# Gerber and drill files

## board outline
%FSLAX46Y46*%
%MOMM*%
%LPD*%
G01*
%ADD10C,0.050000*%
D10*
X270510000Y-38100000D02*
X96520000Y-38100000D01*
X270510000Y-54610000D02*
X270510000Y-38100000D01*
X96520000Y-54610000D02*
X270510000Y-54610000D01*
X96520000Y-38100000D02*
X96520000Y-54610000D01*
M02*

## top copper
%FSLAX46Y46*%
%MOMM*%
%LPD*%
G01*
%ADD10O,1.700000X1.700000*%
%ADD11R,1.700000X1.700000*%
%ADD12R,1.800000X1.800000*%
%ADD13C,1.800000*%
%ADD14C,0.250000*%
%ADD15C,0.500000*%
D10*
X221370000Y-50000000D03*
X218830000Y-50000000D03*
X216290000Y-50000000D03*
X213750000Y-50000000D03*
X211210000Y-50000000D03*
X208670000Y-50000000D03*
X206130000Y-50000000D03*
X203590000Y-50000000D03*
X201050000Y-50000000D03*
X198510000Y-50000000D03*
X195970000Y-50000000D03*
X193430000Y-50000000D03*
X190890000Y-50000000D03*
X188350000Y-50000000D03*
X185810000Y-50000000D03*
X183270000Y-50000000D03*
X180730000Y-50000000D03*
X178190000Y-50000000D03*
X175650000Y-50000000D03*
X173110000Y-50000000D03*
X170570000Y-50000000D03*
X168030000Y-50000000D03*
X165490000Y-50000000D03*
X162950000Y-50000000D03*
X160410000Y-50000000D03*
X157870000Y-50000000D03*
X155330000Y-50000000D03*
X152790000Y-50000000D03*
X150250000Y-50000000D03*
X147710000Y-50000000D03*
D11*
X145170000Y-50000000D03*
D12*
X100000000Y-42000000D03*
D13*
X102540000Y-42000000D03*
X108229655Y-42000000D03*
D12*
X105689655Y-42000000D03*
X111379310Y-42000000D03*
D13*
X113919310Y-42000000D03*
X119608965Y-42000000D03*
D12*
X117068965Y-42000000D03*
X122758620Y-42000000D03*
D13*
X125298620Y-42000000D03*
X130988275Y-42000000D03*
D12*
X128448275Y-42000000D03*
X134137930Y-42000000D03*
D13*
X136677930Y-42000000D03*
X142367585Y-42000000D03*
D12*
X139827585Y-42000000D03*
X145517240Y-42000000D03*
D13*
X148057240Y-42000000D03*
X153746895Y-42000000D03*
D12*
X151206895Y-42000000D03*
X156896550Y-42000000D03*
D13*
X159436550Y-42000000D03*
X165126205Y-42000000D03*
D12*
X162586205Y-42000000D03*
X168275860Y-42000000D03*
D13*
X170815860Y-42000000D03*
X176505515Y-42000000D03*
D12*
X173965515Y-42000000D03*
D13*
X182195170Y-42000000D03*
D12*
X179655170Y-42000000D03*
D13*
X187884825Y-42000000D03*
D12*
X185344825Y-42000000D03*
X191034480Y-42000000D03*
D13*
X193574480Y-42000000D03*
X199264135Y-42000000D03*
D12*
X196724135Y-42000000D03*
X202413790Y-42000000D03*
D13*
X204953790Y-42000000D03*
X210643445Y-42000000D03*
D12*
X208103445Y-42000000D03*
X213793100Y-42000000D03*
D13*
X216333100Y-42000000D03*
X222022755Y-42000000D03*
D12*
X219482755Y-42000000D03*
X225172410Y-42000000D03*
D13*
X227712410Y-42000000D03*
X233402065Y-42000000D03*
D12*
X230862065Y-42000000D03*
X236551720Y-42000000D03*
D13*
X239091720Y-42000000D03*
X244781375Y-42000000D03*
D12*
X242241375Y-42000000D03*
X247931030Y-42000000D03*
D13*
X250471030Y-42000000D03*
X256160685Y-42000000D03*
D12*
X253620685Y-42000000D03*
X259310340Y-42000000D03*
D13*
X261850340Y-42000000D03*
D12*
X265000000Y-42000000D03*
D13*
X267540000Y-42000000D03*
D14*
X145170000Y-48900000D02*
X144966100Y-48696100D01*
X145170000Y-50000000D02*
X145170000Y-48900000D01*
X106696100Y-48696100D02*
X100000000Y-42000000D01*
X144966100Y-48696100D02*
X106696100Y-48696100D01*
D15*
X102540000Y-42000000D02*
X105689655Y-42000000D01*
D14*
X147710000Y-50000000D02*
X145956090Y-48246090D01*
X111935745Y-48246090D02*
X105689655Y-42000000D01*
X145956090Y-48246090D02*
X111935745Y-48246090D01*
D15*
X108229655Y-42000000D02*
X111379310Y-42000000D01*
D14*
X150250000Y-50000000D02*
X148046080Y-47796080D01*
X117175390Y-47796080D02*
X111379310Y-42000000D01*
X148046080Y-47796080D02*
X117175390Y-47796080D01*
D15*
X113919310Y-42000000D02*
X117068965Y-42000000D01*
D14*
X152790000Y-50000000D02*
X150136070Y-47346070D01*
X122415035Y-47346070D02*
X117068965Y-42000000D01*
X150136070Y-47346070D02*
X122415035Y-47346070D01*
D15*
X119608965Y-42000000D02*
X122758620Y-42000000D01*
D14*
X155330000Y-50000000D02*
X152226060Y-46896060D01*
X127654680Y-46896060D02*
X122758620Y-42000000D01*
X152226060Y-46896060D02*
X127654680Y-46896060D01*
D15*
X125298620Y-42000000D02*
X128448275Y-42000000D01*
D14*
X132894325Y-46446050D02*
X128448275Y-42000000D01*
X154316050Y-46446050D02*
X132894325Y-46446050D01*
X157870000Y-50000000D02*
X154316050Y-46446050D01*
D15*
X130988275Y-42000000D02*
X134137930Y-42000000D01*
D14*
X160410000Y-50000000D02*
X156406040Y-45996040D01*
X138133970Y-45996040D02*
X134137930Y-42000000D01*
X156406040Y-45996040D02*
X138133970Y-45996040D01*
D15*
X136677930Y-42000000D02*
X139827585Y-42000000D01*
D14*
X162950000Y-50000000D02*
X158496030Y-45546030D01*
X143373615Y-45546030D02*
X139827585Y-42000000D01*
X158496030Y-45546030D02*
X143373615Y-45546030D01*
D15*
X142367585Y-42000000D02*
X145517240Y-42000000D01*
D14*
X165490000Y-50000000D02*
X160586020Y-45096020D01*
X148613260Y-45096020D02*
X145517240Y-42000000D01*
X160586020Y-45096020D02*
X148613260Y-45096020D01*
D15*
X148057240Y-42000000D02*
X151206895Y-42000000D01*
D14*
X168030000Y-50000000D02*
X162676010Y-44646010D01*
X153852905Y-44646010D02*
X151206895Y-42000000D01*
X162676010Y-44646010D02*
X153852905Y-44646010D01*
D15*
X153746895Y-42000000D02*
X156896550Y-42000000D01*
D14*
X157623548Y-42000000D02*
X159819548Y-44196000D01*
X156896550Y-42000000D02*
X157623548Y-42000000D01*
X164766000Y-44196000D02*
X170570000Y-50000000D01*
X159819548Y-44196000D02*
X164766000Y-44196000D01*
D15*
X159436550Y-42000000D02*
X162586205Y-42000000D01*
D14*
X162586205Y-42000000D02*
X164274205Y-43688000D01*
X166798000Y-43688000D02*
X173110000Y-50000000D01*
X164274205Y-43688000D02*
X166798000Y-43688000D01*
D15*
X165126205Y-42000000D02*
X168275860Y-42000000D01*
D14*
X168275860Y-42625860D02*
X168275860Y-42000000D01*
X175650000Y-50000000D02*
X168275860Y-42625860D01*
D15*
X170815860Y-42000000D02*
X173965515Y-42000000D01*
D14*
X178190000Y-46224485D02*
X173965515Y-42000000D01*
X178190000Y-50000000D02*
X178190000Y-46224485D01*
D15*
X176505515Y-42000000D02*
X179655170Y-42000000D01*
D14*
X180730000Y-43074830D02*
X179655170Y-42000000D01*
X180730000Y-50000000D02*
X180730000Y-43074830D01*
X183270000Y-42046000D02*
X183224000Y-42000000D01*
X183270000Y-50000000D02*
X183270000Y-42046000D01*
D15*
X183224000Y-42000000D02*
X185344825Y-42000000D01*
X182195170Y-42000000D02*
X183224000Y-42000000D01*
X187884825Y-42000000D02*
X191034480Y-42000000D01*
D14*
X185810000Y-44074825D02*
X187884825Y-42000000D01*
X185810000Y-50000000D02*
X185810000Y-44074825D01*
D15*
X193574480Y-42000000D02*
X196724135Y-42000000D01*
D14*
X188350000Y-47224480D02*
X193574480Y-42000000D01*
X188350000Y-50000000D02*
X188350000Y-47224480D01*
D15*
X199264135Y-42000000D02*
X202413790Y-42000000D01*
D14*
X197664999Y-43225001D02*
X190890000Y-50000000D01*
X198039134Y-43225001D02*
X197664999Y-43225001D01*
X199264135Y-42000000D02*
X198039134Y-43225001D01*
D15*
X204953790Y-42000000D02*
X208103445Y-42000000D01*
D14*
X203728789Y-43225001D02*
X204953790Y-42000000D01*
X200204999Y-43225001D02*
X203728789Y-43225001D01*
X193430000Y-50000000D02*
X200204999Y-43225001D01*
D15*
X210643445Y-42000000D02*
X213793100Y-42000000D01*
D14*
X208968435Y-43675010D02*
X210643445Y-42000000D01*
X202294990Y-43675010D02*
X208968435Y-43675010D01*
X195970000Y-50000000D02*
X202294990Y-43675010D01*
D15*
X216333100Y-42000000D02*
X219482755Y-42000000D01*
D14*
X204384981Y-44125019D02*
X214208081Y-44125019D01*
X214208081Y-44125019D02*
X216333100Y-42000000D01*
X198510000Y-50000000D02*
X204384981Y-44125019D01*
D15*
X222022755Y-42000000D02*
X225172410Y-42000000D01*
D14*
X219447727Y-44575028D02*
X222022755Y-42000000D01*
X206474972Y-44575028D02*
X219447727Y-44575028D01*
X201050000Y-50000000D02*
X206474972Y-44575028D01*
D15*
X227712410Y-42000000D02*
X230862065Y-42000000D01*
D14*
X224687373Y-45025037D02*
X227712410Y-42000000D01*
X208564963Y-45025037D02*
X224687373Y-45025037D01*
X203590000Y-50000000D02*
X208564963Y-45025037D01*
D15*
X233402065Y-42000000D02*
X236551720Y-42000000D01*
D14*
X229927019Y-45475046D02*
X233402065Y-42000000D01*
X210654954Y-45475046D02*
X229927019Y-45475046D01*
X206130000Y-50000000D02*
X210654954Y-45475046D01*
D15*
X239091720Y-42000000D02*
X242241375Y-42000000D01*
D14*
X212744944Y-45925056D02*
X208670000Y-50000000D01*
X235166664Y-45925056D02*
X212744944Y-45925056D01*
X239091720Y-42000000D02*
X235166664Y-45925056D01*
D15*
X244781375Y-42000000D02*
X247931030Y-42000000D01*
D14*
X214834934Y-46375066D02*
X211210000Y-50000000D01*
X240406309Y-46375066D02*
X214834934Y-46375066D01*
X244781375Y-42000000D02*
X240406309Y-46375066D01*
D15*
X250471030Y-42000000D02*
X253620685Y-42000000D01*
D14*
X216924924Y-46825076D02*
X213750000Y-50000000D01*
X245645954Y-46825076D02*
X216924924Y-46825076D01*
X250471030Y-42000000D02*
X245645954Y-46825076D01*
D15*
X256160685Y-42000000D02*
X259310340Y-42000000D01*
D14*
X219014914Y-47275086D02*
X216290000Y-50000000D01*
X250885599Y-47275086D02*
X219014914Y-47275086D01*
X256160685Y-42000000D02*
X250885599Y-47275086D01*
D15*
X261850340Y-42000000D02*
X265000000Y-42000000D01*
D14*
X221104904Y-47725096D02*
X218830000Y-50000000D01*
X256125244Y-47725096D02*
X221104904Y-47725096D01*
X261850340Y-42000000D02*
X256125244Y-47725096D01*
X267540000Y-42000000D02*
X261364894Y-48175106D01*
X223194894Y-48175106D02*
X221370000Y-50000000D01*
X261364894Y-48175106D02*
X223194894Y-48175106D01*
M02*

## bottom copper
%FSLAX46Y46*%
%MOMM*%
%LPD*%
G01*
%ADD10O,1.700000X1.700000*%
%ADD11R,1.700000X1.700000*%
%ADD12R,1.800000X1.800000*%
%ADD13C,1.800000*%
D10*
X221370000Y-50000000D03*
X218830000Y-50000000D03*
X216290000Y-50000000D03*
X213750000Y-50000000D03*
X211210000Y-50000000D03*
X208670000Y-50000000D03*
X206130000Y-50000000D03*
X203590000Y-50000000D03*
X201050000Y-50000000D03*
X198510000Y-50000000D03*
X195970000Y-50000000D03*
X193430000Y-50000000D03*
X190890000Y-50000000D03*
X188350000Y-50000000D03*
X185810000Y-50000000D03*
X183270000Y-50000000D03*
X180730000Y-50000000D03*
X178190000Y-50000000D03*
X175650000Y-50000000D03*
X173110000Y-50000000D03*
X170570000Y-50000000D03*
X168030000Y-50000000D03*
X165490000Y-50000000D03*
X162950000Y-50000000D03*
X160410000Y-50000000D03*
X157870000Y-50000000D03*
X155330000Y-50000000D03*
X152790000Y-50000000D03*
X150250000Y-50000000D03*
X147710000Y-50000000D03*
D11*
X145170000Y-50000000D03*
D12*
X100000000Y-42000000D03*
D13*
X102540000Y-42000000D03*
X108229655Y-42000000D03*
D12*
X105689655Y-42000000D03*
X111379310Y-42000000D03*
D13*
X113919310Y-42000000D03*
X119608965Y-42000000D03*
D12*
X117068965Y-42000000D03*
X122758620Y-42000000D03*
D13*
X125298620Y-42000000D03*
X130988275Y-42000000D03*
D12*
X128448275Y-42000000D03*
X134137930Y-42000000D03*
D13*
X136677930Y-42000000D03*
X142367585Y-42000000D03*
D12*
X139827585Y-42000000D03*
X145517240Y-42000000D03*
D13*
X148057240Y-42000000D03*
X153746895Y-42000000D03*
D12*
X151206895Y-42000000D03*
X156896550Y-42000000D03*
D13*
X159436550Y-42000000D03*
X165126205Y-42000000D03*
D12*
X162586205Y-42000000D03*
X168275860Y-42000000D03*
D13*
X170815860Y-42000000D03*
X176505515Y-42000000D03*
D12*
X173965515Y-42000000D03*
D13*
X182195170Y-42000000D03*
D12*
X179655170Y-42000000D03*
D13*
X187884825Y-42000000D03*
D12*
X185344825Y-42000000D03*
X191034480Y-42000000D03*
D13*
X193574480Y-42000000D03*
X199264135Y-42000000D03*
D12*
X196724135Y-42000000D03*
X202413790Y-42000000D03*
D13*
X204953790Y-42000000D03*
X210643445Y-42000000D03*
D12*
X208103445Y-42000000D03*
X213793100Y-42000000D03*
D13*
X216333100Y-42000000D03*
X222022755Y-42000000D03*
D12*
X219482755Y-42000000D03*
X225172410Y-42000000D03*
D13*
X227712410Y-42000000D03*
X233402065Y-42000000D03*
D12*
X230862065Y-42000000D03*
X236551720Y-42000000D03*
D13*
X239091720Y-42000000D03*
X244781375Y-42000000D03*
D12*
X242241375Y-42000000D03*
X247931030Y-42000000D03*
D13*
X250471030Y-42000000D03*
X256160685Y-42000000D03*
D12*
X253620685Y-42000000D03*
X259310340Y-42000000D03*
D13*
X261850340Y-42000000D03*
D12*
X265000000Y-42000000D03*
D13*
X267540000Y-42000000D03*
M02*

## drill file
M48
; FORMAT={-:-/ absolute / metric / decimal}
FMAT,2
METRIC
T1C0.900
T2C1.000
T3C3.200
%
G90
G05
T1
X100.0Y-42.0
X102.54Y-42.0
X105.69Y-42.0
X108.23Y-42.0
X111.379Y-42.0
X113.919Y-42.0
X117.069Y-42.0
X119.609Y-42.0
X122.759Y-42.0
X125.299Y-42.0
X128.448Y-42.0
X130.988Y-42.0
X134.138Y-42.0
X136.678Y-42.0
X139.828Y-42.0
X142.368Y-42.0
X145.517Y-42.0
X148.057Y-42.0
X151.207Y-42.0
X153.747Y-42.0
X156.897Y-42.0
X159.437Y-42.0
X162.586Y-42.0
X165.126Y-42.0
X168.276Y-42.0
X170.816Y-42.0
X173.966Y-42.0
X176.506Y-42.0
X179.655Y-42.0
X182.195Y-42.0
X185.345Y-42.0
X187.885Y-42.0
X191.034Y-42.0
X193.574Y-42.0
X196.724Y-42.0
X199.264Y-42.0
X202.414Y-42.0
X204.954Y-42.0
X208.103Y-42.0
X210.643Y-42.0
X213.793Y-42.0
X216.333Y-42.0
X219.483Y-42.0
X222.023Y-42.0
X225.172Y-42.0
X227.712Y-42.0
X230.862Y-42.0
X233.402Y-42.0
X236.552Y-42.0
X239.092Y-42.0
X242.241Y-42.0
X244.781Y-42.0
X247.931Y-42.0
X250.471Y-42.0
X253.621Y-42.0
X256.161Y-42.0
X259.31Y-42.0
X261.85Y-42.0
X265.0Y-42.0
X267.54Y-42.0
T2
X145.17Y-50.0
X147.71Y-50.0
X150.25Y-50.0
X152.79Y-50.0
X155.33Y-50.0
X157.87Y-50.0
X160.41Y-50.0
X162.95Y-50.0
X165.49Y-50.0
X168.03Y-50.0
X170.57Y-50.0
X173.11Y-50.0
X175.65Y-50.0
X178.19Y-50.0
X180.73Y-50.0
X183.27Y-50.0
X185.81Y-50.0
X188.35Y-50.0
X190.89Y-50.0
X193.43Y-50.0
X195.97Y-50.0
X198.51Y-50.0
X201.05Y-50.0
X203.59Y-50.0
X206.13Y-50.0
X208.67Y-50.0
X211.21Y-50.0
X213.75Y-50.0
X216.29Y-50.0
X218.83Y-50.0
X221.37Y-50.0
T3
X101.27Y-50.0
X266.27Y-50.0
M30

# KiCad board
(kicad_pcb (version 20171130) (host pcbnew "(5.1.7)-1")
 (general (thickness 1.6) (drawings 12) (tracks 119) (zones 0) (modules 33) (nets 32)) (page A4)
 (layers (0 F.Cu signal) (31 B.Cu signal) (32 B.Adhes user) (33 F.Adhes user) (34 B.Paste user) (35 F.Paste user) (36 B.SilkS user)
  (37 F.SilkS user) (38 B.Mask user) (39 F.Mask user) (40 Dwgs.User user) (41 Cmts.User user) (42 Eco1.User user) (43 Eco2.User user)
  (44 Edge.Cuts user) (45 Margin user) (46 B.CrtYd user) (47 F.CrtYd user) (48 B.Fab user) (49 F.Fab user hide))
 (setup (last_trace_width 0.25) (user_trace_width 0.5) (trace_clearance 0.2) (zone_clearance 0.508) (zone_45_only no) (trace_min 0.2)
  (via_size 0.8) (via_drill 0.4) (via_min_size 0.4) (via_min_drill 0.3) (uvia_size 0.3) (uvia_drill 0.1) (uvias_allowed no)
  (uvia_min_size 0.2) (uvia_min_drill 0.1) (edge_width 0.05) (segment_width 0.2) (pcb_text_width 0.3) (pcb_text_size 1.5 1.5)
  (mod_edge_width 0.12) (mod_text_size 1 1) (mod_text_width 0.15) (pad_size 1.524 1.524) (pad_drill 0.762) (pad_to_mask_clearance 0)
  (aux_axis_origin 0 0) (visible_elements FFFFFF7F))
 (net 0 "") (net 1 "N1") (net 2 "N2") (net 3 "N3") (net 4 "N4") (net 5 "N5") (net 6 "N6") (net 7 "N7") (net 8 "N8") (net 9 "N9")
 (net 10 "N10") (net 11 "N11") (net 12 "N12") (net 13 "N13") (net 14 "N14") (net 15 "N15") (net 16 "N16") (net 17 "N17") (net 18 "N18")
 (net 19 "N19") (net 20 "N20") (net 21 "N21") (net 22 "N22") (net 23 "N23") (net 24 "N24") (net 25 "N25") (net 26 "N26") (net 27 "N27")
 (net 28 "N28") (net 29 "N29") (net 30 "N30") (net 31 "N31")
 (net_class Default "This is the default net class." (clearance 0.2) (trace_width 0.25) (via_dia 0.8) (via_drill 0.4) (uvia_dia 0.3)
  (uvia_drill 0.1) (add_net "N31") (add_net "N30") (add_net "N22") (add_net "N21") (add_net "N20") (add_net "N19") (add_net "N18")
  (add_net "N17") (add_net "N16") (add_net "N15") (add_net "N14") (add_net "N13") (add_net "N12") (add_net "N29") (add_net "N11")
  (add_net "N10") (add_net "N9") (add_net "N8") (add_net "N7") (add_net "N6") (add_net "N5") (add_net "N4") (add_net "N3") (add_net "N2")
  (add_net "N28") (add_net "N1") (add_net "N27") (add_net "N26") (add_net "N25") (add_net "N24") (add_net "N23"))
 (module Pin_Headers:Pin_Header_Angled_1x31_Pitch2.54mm (layer F.Cu) (at 145.17 50 90)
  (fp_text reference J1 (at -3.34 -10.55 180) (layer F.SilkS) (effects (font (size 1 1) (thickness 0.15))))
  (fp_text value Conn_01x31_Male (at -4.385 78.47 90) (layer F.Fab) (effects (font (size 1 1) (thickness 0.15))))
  (pad 31 thru_hole oval (at 0 76.2 90) (size 1.7 1.7) (drill 1) (layers *.Cu *.Mask) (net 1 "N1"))
  (pad 30 thru_hole oval (at 0 73.66 90) (size 1.7 1.7) (drill 1) (layers *.Cu *.Mask) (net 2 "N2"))
  (pad 29 thru_hole oval (at 0 71.12 90) (size 1.7 1.7) (drill 1) (layers *.Cu *.Mask) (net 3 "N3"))
  (pad 28 thru_hole oval (at 0 68.58 90) (size 1.7 1.7) (drill 1) (layers *.Cu *.Mask) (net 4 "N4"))
  (pad 27 thru_hole oval (at 0 66.04 90) (size 1.7 1.7) (drill 1) (layers *.Cu *.Mask) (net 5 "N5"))
  (pad 26 thru_hole oval (at 0 63.5 90) (size 1.7 1.7) (drill 1) (layers *.Cu *.Mask) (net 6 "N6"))
  (pad 25 thru_hole oval (at 0 60.96 90) (size 1.7 1.7) (drill 1) (layers *.Cu *.Mask) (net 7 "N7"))
  (pad 24 thru_hole oval (at 0 58.42 90) (size 1.7 1.7) (drill 1) (layers *.Cu *.Mask) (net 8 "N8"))
  (pad 23 thru_hole oval (at 0 55.88 90) (size 1.7 1.7) (drill 1) (layers *.Cu *.Mask) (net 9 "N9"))
  (pad 22 thru_hole oval (at 0 53.34 90) (size 1.7 1.7) (drill 1) (layers *.Cu *.Mask) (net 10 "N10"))
  (pad 21 thru_hole oval (at 0 50.8 90) (size 1.7 1.7) (drill 1) (layers *.Cu *.Mask) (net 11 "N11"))
  (pad 20 thru_hole oval (at 0 48.26 90) (size 1.7 1.7) (drill 1) (layers *.Cu *.Mask) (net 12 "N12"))
  (pad 19 thru_hole oval (at 0 45.72 90) (size 1.7 1.7) (drill 1) (layers *.Cu *.Mask) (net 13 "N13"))
  (pad 18 thru_hole oval (at 0 43.18 90) (size 1.7 1.7) (drill 1) (layers *.Cu *.Mask) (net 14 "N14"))
  (pad 17 thru_hole oval (at 0 40.64 90) (size 1.7 1.7) (drill 1) (layers *.Cu *.Mask) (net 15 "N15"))
  (pad 16 thru_hole oval (at 0 38.1 90) (size 1.7 1.7) (drill 1) (layers *.Cu *.Mask) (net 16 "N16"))
  (pad 15 thru_hole oval (at 0 35.56 90) (size 1.7 1.7) (drill 1) (layers *.Cu *.Mask) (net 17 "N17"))
  (pad 14 thru_hole oval (at 0 33.02 90) (size 1.7 1.7) (drill 1) (layers *.Cu *.Mask) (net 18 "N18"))
  (pad 13 thru_hole oval (at 0 30.48 90) (size 1.7 1.7) (drill 1) (layers *.Cu *.Mask) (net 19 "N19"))
  (pad 12 thru_hole oval (at 0 27.94 90) (size 1.7 1.7) (drill 1) (layers *.Cu *.Mask) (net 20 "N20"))
  (pad 11 thru_hole oval (at 0 25.4 90) (size 1.7 1.7) (drill 1) (layers *.Cu *.Mask) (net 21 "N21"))
  (pad 10 thru_hole oval (at 0 22.86 90) (size 1.7 1.7) (drill 1) (layers *.Cu *.Mask) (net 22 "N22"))
  (pad 9 thru_hole oval (at 0 20.32 90) (size 1.7 1.7) (drill 1) (layers *.Cu *.Mask) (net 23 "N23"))
  (pad 8 thru_hole oval (at 0 17.78 90) (size 1.7 1.7) (drill 1) (layers *.Cu *.Mask) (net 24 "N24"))
  (pad 7 thru_hole oval (at 0 15.24 90) (size 1.7 1.7) (drill 1) (layers *.Cu *.Mask) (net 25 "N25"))
  (pad 6 thru_hole oval (at 0 12.7 90) (size 1.7 1.7) (drill 1) (layers *.Cu *.Mask) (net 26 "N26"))
  (pad 5 thru_hole oval (at 0 10.16 90) (size 1.7 1.7) (drill 1) (layers *.Cu *.Mask) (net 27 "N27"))
  (pad 4 thru_hole oval (at 0 7.62 90) (size 1.7 1.7) (drill 1) (layers *.Cu *.Mask) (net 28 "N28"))
  (pad 3 thru_hole oval (at 0 5.08 90) (size 1.7 1.7) (drill 1) (layers *.Cu *.Mask) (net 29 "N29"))
  (pad 2 thru_hole oval (at 0 2.54 90) (size 1.7 1.7) (drill 1) (layers *.Cu *.Mask) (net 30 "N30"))
  (pad 1 thru_hole rect (at 0 0 90) (size 1.7 1.7) (drill 1) (layers *.Cu *.Mask) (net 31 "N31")))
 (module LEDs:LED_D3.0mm (layer F.Cu) (at 100 42)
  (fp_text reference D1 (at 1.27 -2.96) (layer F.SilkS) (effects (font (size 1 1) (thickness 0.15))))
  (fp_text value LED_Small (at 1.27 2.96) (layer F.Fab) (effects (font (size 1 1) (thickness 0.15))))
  (pad 1 thru_hole rect (at 0 0) (size 1.8 1.8) (drill 0.9) (layers *.Cu *.Mask) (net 31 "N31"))
  (pad 2 thru_hole circle (at 2.54 0) (size 1.8 1.8) (drill 0.9) (layers *.Cu *.Mask) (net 30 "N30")))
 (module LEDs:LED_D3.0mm (layer F.Cu) (at 105.689655 42)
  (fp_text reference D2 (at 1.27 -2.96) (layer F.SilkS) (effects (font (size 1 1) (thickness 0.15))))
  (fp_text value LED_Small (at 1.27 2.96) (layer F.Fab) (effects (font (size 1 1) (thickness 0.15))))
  (pad 2 thru_hole circle (at 2.54 0) (size 1.8 1.8) (drill 0.9) (layers *.Cu *.Mask) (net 29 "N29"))
  (pad 1 thru_hole rect (at 0 0) (size 1.8 1.8) (drill 0.9) (layers *.Cu *.Mask) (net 30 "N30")))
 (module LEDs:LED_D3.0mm (layer F.Cu) (at 111.37931 42)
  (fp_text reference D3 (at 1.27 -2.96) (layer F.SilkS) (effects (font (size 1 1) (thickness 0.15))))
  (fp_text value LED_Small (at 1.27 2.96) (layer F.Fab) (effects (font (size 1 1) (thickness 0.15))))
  (pad 1 thru_hole rect (at 0 0) (size 1.8 1.8) (drill 0.9) (layers *.Cu *.Mask) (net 29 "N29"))
  (pad 2 thru_hole circle (at 2.54 0) (size 1.8 1.8) (drill 0.9) (layers *.Cu *.Mask) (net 28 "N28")))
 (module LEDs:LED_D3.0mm (layer F.Cu) (at 117.068965 42)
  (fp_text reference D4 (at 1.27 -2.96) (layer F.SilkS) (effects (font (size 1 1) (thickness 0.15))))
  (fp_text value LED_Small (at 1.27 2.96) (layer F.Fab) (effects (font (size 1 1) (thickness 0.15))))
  (pad 2 thru_hole circle (at 2.54 0) (size 1.8 1.8) (drill 0.9) (layers *.Cu *.Mask) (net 27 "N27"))
  (pad 1 thru_hole rect (at 0 0) (size 1.8 1.8) (drill 0.9) (layers *.Cu *.Mask) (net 28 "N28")))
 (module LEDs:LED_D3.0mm (layer F.Cu) (at 122.75862 42)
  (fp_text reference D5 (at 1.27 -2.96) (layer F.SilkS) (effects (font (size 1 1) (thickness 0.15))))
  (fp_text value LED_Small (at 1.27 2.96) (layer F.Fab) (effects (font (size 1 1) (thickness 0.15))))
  (pad 1 thru_hole rect (at 0 0) (size 1.8 1.8) (drill 0.9) (layers *.Cu *.Mask) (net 27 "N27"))
  (pad 2 thru_hole circle (at 2.54 0) (size 1.8 1.8) (drill 0.9) (layers *.Cu *.Mask) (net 26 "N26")))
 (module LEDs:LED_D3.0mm (layer F.Cu) (at 128.448275 42)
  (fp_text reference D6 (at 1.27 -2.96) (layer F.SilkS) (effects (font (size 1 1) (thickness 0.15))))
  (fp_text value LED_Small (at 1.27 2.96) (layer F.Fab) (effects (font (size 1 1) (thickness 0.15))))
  (pad 2 thru_hole circle (at 2.54 0) (size 1.8 1.8) (drill 0.9) (layers *.Cu *.Mask) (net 25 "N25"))
  (pad 1 thru_hole rect (at 0 0) (size 1.8 1.8) (drill 0.9) (layers *.Cu *.Mask) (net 26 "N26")))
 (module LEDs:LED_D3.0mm (layer F.Cu) (at 134.13793 42)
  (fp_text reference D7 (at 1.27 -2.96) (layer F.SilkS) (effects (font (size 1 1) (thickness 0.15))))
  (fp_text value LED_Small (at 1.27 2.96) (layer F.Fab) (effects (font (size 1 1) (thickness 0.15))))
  (pad 1 thru_hole rect (at 0 0) (size 1.8 1.8) (drill 0.9) (layers *.Cu *.Mask) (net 25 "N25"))
  (pad 2 thru_hole circle (at 2.54 0) (size 1.8 1.8) (drill 0.9) (layers *.Cu *.Mask) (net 24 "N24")))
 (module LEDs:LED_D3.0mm (layer F.Cu) (at 139.827585 42)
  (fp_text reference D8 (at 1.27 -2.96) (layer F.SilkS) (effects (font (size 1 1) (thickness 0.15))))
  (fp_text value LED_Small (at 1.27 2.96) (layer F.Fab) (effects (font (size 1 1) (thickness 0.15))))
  (pad 2 thru_hole circle (at 2.54 0) (size 1.8 1.8) (drill 0.9) (layers *.Cu *.Mask) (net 23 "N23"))
  (pad 1 thru_hole rect (at 0 0) (size 1.8 1.8) (drill 0.9) (layers *.Cu *.Mask) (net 24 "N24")))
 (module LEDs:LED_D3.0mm (layer F.Cu) (at 145.51724 42)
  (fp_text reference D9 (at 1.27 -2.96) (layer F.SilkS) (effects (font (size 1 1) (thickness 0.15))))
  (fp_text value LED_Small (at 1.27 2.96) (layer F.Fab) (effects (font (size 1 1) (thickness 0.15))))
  (pad 1 thru_hole rect (at 0 0) (size 1.8 1.8) (drill 0.9) (layers *.Cu *.Mask) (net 23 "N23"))
  (pad 2 thru_hole circle (at 2.54 0) (size 1.8 1.8) (drill 0.9) (layers *.Cu *.Mask) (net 22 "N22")))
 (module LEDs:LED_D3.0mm (layer F.Cu) (at 151.206895 42)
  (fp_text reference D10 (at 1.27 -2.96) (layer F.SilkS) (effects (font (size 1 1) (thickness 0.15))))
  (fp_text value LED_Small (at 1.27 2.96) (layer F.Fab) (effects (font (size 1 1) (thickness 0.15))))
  (pad 2 thru_hole circle (at 2.54 0) (size 1.8 1.8) (drill 0.9) (layers *.Cu *.Mask) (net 21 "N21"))
  (pad 1 thru_hole rect (at 0 0) (size 1.8 1.8) (drill 0.9) (layers *.Cu *.Mask) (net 22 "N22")))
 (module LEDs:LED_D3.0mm (layer F.Cu) (at 156.89655 42)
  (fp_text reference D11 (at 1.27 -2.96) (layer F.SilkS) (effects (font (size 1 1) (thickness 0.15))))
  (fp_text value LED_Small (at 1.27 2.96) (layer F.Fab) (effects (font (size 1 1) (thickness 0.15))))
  (pad 1 thru_hole rect (at 0 0) (size 1.8 1.8) (drill 0.9) (layers *.Cu *.Mask) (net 21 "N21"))
  (pad 2 thru_hole circle (at 2.54 0) (size 1.8 1.8) (drill 0.9) (layers *.Cu *.Mask) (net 20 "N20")))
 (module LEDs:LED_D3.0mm (layer F.Cu) (at 162.586205 42)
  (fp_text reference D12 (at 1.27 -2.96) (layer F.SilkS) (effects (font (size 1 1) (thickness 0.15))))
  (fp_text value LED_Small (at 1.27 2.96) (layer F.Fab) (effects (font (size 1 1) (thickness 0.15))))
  (pad 2 thru_hole circle (at 2.54 0) (size 1.8 1.8) (drill 0.9) (layers *.Cu *.Mask) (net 19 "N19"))
  (pad 1 thru_hole rect (at 0 0) (size 1.8 1.8) (drill 0.9) (layers *.Cu *.Mask) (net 20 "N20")))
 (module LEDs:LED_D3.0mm (layer F.Cu) (at 168.27586 42)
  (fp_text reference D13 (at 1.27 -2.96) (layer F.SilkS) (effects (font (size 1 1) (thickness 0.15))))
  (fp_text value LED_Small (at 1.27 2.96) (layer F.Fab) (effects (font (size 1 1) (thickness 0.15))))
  (pad 1 thru_hole rect (at 0 0) (size 1.8 1.8) (drill 0.9) (layers *.Cu *.Mask) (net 19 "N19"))
  (pad 2 thru_hole circle (at 2.54 0) (size 1.8 1.8) (drill 0.9) (layers *.Cu *.Mask) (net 18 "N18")))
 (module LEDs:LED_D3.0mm (layer F.Cu) (at 173.965515 42)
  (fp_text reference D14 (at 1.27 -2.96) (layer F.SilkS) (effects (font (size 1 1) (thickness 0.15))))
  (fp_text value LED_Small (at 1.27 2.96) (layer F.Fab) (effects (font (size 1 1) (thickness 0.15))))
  (pad 2 thru_hole circle (at 2.54 0) (size 1.8 1.8) (drill 0.9) (layers *.Cu *.Mask) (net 17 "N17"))
  (pad 1 thru_hole rect (at 0 0) (size 1.8 1.8) (drill 0.9) (layers *.Cu *.Mask) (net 18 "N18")))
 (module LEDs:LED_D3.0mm (layer F.Cu) (at 179.65517 42)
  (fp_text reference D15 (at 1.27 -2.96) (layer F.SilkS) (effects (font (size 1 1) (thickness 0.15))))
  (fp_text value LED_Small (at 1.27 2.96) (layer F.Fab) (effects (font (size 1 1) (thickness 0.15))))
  (pad 2 thru_hole circle (at 2.54 0) (size 1.8 1.8) (drill 0.9) (layers *.Cu *.Mask) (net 16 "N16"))
  (pad 1 thru_hole rect (at 0 0) (size 1.8 1.8) (drill 0.9) (layers *.Cu *.Mask) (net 17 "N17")))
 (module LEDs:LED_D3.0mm (layer F.Cu) (at 185.344825 42)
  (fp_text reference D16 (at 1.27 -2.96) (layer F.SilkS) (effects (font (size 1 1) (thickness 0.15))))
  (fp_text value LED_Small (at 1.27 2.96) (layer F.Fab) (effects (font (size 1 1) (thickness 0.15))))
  (pad 2 thru_hole circle (at 2.54 0) (size 1.8 1.8) (drill 0.9) (layers *.Cu *.Mask) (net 15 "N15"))
  (pad 1 thru_hole rect (at 0 0) (size 1.8 1.8) (drill 0.9) (layers *.Cu *.Mask) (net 16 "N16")))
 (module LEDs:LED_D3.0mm (layer F.Cu) (at 191.03448 42)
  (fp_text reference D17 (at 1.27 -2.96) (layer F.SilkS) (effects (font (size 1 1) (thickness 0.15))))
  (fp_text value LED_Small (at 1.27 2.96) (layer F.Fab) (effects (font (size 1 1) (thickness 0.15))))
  (pad 1 thru_hole rect (at 0 0) (size 1.8 1.8) (drill 0.9) (layers *.Cu *.Mask) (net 15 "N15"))
  (pad 2 thru_hole circle (at 2.54 0) (size 1.8 1.8) (drill 0.9) (layers *.Cu *.Mask) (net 14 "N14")))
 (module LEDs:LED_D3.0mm (layer F.Cu) (at 196.724135 42)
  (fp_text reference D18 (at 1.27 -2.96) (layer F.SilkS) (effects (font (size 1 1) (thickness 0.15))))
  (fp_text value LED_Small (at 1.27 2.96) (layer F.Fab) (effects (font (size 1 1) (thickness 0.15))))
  (pad 2 thru_hole circle (at 2.54 0) (size 1.8 1.8) (drill 0.9) (layers *.Cu *.Mask) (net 13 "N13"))
  (pad 1 thru_hole rect (at 0 0) (size 1.8 1.8) (drill 0.9) (layers *.Cu *.Mask) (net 14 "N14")))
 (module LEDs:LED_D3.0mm (layer F.Cu) (at 202.41379 42)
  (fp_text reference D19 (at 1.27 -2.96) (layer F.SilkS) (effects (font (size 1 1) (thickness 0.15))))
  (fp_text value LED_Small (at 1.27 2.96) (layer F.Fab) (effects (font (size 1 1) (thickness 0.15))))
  (pad 1 thru_hole rect (at 0 0) (size 1.8 1.8) (drill 0.9) (layers *.Cu *.Mask) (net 13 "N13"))
  (pad 2 thru_hole circle (at 2.54 0) (size 1.8 1.8) (drill 0.9) (layers *.Cu *.Mask) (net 12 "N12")))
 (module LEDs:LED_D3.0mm (layer F.Cu) (at 208.103445 42)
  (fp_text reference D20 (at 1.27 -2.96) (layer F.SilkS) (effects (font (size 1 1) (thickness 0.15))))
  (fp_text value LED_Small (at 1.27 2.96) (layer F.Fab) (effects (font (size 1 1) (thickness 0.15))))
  (pad 2 thru_hole circle (at 2.54 0) (size 1.8 1.8) (drill 0.9) (layers *.Cu *.Mask) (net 11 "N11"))
  (pad 1 thru_hole rect (at 0 0) (size 1.8 1.8) (drill 0.9) (layers *.Cu *.Mask) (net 12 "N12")))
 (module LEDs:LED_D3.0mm (layer F.Cu) (at 213.7931 42)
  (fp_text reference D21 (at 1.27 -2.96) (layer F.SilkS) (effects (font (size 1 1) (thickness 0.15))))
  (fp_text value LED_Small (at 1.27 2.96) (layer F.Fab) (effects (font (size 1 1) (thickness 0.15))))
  (pad 1 thru_hole rect (at 0 0) (size 1.8 1.8) (drill 0.9) (layers *.Cu *.Mask) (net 11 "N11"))
  (pad 2 thru_hole circle (at 2.54 0) (size 1.8 1.8) (drill 0.9) (layers *.Cu *.Mask) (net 10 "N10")))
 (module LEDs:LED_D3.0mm (layer F.Cu) (at 219.482755 42)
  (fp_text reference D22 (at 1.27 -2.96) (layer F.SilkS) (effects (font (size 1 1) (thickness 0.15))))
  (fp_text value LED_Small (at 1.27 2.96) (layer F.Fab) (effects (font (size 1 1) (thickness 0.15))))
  (pad 2 thru_hole circle (at 2.54 0) (size 1.8 1.8) (drill 0.9) (layers *.Cu *.Mask) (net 9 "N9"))
  (pad 1 thru_hole rect (at 0 0) (size 1.8 1.8) (drill 0.9) (layers *.Cu *.Mask) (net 10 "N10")))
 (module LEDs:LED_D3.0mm (layer F.Cu) (at 225.17241 42)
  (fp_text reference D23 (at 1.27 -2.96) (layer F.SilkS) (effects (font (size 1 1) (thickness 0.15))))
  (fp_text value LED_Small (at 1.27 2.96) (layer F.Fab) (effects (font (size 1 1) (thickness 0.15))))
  (pad 1 thru_hole rect (at 0 0) (size 1.8 1.8) (drill 0.9) (layers *.Cu *.Mask) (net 9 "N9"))
  (pad 2 thru_hole circle (at 2.54 0) (size 1.8 1.8) (drill 0.9) (layers *.Cu *.Mask) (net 8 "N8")))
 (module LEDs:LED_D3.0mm (layer F.Cu) (at 230.862065 42)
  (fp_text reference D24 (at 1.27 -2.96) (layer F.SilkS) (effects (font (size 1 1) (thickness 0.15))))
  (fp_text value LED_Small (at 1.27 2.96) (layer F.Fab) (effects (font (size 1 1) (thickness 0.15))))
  (pad 2 thru_hole circle (at 2.54 0) (size 1.8 1.8) (drill 0.9) (layers *.Cu *.Mask) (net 7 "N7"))
  (pad 1 thru_hole rect (at 0 0) (size 1.8 1.8) (drill 0.9) (layers *.Cu *.Mask) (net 8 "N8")))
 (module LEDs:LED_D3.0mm (layer F.Cu) (at 236.55172 42)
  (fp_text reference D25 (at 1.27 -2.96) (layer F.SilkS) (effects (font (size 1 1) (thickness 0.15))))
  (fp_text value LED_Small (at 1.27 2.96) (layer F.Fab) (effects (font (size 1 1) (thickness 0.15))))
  (pad 1 thru_hole rect (at 0 0) (size 1.8 1.8) (drill 0.9) (layers *.Cu *.Mask) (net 7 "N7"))
  (pad 2 thru_hole circle (at 2.54 0) (size 1.8 1.8) (drill 0.9) (layers *.Cu *.Mask) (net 6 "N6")))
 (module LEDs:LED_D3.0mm (layer F.Cu) (at 242.241375 42)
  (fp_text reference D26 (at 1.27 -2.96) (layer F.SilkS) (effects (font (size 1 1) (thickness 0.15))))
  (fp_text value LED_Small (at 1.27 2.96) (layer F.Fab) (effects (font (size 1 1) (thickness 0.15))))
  (pad 2 thru_hole circle (at 2.54 0) (size 1.8 1.8) (drill 0.9) (layers *.Cu *.Mask) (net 5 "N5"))
  (pad 1 thru_hole rect (at 0 0) (size 1.8 1.8) (drill 0.9) (layers *.Cu *.Mask) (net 6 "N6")))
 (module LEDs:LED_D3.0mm (layer F.Cu) (at 247.93103 42)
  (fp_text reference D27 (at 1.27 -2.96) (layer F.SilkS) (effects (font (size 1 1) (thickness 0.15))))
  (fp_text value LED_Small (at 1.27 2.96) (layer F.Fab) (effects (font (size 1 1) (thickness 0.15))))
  (pad 1 thru_hole rect (at 0 0) (size 1.8 1.8) (drill 0.9) (layers *.Cu *.Mask) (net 5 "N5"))
  (pad 2 thru_hole circle (at 2.54 0) (size 1.8 1.8) (drill 0.9) (layers *.Cu *.Mask) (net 4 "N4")))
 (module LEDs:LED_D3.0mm (layer F.Cu) (at 253.620685 42)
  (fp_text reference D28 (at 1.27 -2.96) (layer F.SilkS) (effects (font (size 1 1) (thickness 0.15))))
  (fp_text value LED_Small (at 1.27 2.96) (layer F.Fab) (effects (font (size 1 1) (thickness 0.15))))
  (pad 2 thru_hole circle (at 2.54 0) (size 1.8 1.8) (drill 0.9) (layers *.Cu *.Mask) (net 3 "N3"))
  (pad 1 thru_hole rect (at 0 0) (size 1.8 1.8) (drill 0.9) (layers *.Cu *.Mask) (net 4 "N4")))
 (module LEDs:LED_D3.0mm (layer F.Cu) (at 259.31034 42)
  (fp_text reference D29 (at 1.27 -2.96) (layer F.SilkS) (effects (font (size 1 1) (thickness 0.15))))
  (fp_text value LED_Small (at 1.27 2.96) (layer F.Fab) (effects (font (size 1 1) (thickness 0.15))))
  (pad 1 thru_hole rect (at 0 0) (size 1.8 1.8) (drill 0.9) (layers *.Cu *.Mask) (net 3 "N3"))
  (pad 2 thru_hole circle (at 2.54 0) (size 1.8 1.8) (drill 0.9) (layers *.Cu *.Mask) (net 2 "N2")))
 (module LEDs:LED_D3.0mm (layer F.Cu) (at 265 42)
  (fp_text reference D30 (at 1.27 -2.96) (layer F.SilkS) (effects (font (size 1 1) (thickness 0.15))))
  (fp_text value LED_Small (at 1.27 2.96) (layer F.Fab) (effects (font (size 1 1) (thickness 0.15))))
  (pad 1 thru_hole rect (at 0 0) (size 1.8 1.8) (drill 0.9) (layers *.Cu *.Mask) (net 2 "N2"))
  (pad 2 thru_hole circle (at 2.54 0) (size 1.8 1.8) (drill 0.9) (layers *.Cu *.Mask) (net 1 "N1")))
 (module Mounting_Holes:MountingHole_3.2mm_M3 (layer F.Cu) (at 101.27 50)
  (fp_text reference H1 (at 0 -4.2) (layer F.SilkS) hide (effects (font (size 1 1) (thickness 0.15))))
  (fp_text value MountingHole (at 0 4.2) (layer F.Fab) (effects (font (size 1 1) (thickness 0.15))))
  (pad 1 np_thru_hole circle (at 0 0) (size 3.2 3.2) (drill 3.2) (layers *.Cu *.Mask)))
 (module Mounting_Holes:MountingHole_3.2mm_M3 (layer F.Cu) (at 266.27 50)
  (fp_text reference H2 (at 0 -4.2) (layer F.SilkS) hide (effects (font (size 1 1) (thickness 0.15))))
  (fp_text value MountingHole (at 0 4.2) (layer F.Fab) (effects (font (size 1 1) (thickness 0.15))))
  (pad 1 np_thru_hole circle (at 0 0) (size 3.2 3.2) (drill 3.2) (layers *.Cu *.Mask)))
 (gr_line (start 270.51 38.1) (end 96.52 38.1) (layer Edge.Cuts) (width 0.05))
 (gr_line (start 270.51 54.61) (end 270.51 38.1) (layer Edge.Cuts) (width 0.05))
 (gr_line (start 96.52 54.61) (end 270.51 54.61) (layer Edge.Cuts) (width 0.05))
 (gr_line (start 96.52 38.1) (end 96.52 54.61) (layer Edge.Cuts) (width 0.05))
 (segment (start 145.17 48.9) (end 144.9661 48.6961) (width 0.25) (layer F.Cu) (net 31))
 (segment (start 145.17 50) (end 145.17 48.9) (width 0.25) (layer F.Cu) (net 31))
 (segment (start 106.6961 48.6961) (end 100 42) (width 0.25) (layer F.Cu) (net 31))
 (segment (start 144.9661 48.6961) (end 106.6961 48.6961) (width 0.25) (layer F.Cu) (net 31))
 (segment (start 102.54 42) (end 105.689655 42) (width 0.5) (layer F.Cu) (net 30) (status 30))
 (segment (start 147.71 50) (end 145.95609 48.24609) (width 0.25) (layer F.Cu) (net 30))
 (segment (start 111.935745 48.24609) (end 105.689655 42) (width 0.25) (layer F.Cu) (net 30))
 (segment (start 145.95609 48.24609) (end 111.935745 48.24609) (width 0.25) (layer F.Cu) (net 30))
 (segment (start 108.229655 42) (end 111.37931 42) (width 0.5) (layer F.Cu) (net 29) (status 30))
 (segment (start 150.25 50) (end 148.04608 47.79608) (width 0.25) (layer F.Cu) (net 29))
 (segment (start 117.17539 47.79608) (end 111.37931 42) (width 0.25) (layer F.Cu) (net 29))
 (segment (start 148.04608 47.79608) (end 117.17539 47.79608) (width 0.25) (layer F.Cu) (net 29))
 (segment (start 113.91931 42) (end 117.068965 42) (width 0.5) (layer F.Cu) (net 28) (status 30))
 (segment (start 152.79 50) (end 150.13607 47.34607) (width 0.25) (layer F.Cu) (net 28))
 (segment (start 122.415035 47.34607) (end 117.068965 42) (width 0.25) (layer F.Cu) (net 28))
 (segment (start 150.13607 47.34607) (end 122.415035 47.34607) (width 0.25) (layer F.Cu) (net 28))
 (segment (start 119.608965 42) (end 122.75862 42) (width 0.5) (layer F.Cu) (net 27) (status 30))
 (segment (start 155.33 50) (end 152.22606 46.89606) (width 0.25) (layer F.Cu) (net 27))
 (segment (start 127.65468 46.89606) (end 122.75862 42) (width 0.25) (layer F.Cu) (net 27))
 (segment (start 152.22606 46.89606) (end 127.65468 46.89606) (width 0.25) (layer F.Cu) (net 27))
 (segment (start 125.29862 42) (end 128.448275 42) (width 0.5) (layer F.Cu) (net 26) (status 30))
 (segment (start 132.894325 46.44605) (end 128.448275 42) (width 0.25) (layer F.Cu) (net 26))
 (segment (start 154.31605 46.44605) (end 132.894325 46.44605) (width 0.25) (layer F.Cu) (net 26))
 (segment (start 157.87 50) (end 154.31605 46.44605) (width 0.25) (layer F.Cu) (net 26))
 (segment (start 130.988275 42) (end 134.13793 42) (width 0.5) (layer F.Cu) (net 25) (status 30))
 (segment (start 160.41 50) (end 156.40604 45.99604) (width 0.25) (layer F.Cu) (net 25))
 (segment (start 138.13397 45.99604) (end 134.13793 42) (width 0.25) (layer F.Cu) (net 25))
 (segment (start 156.40604 45.99604) (end 138.13397 45.99604) (width 0.25) (layer F.Cu) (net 25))
 (segment (start 136.67793 42) (end 139.827585 42) (width 0.5) (layer F.Cu) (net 24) (status 30))
 (segment (start 162.95 50) (end 158.49603 45.54603) (width 0.25) (layer F.Cu) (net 24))
 (segment (start 143.373615 45.54603) (end 139.827585 42) (width 0.25) (layer F.Cu) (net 24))
 (segment (start 158.49603 45.54603) (end 143.373615 45.54603) (width 0.25) (layer F.Cu) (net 24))
 (segment (start 142.367585 42) (end 145.51724 42) (width 0.5) (layer F.Cu) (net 23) (status 30))
 (segment (start 165.49 50) (end 160.58602 45.09602) (width 0.25) (layer F.Cu) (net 23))
 (segment (start 148.61326 45.09602) (end 145.51724 42) (width 0.25) (layer F.Cu) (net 23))
 (segment (start 160.58602 45.09602) (end 148.61326 45.09602) (width 0.25) (layer F.Cu) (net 23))
 (segment (start 148.05724 42) (end 151.206895 42) (width 0.5) (layer F.Cu) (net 22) (status 30))
 (segment (start 168.03 50) (end 162.67601 44.64601) (width 0.25) (layer F.Cu) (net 22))
 (segment (start 153.852905 44.64601) (end 151.206895 42) (width 0.25) (layer F.Cu) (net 22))
 (segment (start 162.67601 44.64601) (end 153.852905 44.64601) (width 0.25) (layer F.Cu) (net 22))
 (segment (start 153.746895 42) (end 156.89655 42) (width 0.5) (layer F.Cu) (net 21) (status 30))
 (segment (start 157.623548 42) (end 159.819548 44.196) (width 0.25) (layer F.Cu) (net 21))
 (segment (start 156.89655 42) (end 157.623548 42) (width 0.25) (layer F.Cu) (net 21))
 (segment (start 164.766 44.196) (end 170.57 50) (width 0.25) (layer F.Cu) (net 21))
 (segment (start 159.819548 44.196) (end 164.766 44.196) (width 0.25) (layer F.Cu) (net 21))
 (segment (start 159.43655 42) (end 162.586205 42) (width 0.5) (layer F.Cu) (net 20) (status 30))
 (segment (start 162.586205 42) (end 164.274205 43.688) (width 0.25) (layer F.Cu) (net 20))
 (segment (start 166.798 43.688) (end 173.11 50) (width 0.25) (layer F.Cu) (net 20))
 (segment (start 164.274205 43.688) (end 166.798 43.688) (width 0.25) (layer F.Cu) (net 20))
 (segment (start 165.126205 42) (end 168.27586 42) (width 0.5) (layer F.Cu) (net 19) (status 30))
 (segment (start 168.27586 42.62586) (end 168.27586 42) (width 0.25) (layer F.Cu) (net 19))
 (segment (start 175.65 50) (end 168.27586 42.62586) (width 0.25) (layer F.Cu) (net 19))
 (segment (start 170.81586 42) (end 173.965515 42) (width 0.5) (layer F.Cu) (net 18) (status 30))
 (segment (start 178.19 46.224485) (end 173.965515 42) (width 0.25) (layer F.Cu) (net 18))
 (segment (start 178.19 50) (end 178.19 46.224485) (width 0.25) (layer F.Cu) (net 18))
 (segment (start 176.505515 42) (end 179.65517 42) (width 0.5) (layer F.Cu) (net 17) (status 30))
 (segment (start 180.73 43.07483) (end 179.65517 42) (width 0.25) (layer F.Cu) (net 17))
 (segment (start 180.73 50) (end 180.73 43.07483) (width 0.25) (layer F.Cu) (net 17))
 (segment (start 183.27 42.046) (end 183.224 42) (width 0.25) (layer F.Cu) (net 16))
 (segment (start 183.27 50) (end 183.27 42.046) (width 0.25) (layer F.Cu) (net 16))
 (segment (start 183.224 42) (end 185.344825 42) (width 0.5) (layer F.Cu) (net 16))
 (segment (start 182.19517 42) (end 183.224 42) (width 0.5) (layer F.Cu) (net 16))
 (segment (start 187.884825 42) (end 191.03448 42) (width 0.5) (layer F.Cu) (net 15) (status 30))
 (segment (start 185.81 44.074825) (end 187.884825 42) (width 0.25) (layer F.Cu) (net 15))
 (segment (start 185.81 50) (end 185.81 44.074825) (width 0.25) (layer F.Cu) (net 15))
 (segment (start 193.57448 42) (end 196.724135 42) (width 0.5) (layer F.Cu) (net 14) (status 30))
 (segment (start 188.35 47.22448) (end 193.57448 42) (width 0.25) (layer F.Cu) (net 14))
 (segment (start 188.35 50) (end 188.35 47.22448) (width 0.25) (layer F.Cu) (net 14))
 (segment (start 199.264135 42) (end 202.41379 42) (width 0.5) (layer F.Cu) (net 13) (status 30))
 (segment (start 197.664999 43.225001) (end 190.89 50) (width 0.25) (layer F.Cu) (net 13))
 (segment (start 198.039134 43.225001) (end 197.664999 43.225001) (width 0.25) (layer F.Cu) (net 13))
 (segment (start 199.264135 42) (end 198.039134 43.225001) (width 0.25) (layer F.Cu) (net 13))
 (segment (start 204.95379 42) (end 208.103445 42) (width 0.5) (layer F.Cu) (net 12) (status 30))
 (segment (start 203.728789 43.225001) (end 204.95379 42) (width 0.25) (layer F.Cu) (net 12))
 (segment (start 200.204999 43.225001) (end 203.728789 43.225001) (width 0.25) (layer F.Cu) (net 12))
 (segment (start 193.43 50) (end 200.204999 43.225001) (width 0.25) (layer F.Cu) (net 12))
 (segment (start 210.643445 42) (end 213.7931 42) (width 0.5) (layer F.Cu) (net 11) (status 30))
 (segment (start 208.968435 43.67501) (end 210.643445 42) (width 0.25) (layer F.Cu) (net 11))
 (segment (start 202.29499 43.67501) (end 208.968435 43.67501) (width 0.25) (layer F.Cu) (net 11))
 (segment (start 195.97 50) (end 202.29499 43.67501) (width 0.25) (layer F.Cu) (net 11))
 (segment (start 216.3331 42) (end 219.482755 42) (width 0.5) (layer F.Cu) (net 10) (status 30))
 (segment (start 204.384981 44.125019) (end 214.208081 44.125019) (width 0.25) (layer F.Cu) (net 10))
 (segment (start 214.208081 44.125019) (end 216.3331 42) (width 0.25) (layer F.Cu) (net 10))
 (segment (start 198.51 50) (end 204.384981 44.125019) (width 0.25) (layer F.Cu) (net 10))
 (segment (start 222.022755 42) (end 225.17241 42) (width 0.5) (layer F.Cu) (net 9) (status 30))
 (segment (start 219.447727 44.575028) (end 222.022755 42) (width 0.25) (layer F.Cu) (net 9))
 (segment (start 206.474972 44.575028) (end 219.447727 44.575028) (width 0.25) (layer F.Cu) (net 9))
 (segment (start 201.05 50) (end 206.474972 44.575028) (width 0.25) (layer F.Cu) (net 9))
 (segment (start 227.71241 42) (end 230.862065 42) (width 0.5) (layer F.Cu) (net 8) (status 30))
 (segment (start 224.687373 45.025037) (end 227.71241 42) (width 0.25) (layer F.Cu) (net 8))
 (segment (start 208.564963 45.025037) (end 224.687373 45.025037) (width 0.25) (layer F.Cu) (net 8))
 (segment (start 203.59 50) (end 208.564963 45.025037) (width 0.25) (layer F.Cu) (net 8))
 (segment (start 233.402065 42) (end 236.55172 42) (width 0.5) (layer F.Cu) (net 7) (status 30))
 (segment (start 229.927019 45.475046) (end 233.402065 42) (width 0.25) (layer F.Cu) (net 7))
 (segment (start 210.654954 45.475046) (end 229.927019 45.475046) (width 0.25) (layer F.Cu) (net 7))
 (segment (start 206.13 50) (end 210.654954 45.475046) (width 0.25) (layer F.Cu) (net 7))
 (segment (start 239.09172 42) (end 242.241375 42) (width 0.5) (layer F.Cu) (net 6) (status 30))
 (segment (start 212.744944 45.925056) (end 208.67 50) (width 0.25) (layer F.Cu) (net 6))
 (segment (start 235.166664 45.925056) (end 212.744944 45.925056) (width 0.25) (layer F.Cu) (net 6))
 (segment (start 239.09172 42) (end 235.166664 45.925056) (width 0.25) (layer F.Cu) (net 6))
 (segment (start 244.781375 42) (end 247.93103 42) (width 0.5) (layer F.Cu) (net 5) (status 30))
 (segment (start 214.834934 46.375066) (end 211.21 50) (width 0.25) (layer F.Cu) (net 5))
 (segment (start 240.406309 46.375066) (end 214.834934 46.375066) (width 0.25) (layer F.Cu) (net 5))
 (segment (start 244.781375 42) (end 240.406309 46.375066) (width 0.25) (layer F.Cu) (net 5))
 (segment (start 250.47103 42) (end 253.620685 42) (width 0.5) (layer F.Cu) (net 4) (status 30))
 (segment (start 216.924924 46.825076) (end 213.75 50) (width 0.25) (layer F.Cu) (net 4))
 (segment (start 245.645954 46.825076) (end 216.924924 46.825076) (width 0.25) (layer F.Cu) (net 4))
 (segment (start 250.47103 42) (end 245.645954 46.825076) (width 0.25) (layer F.Cu) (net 4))
 (segment (start 256.160685 42) (end 259.31034 42) (width 0.5) (layer F.Cu) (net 3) (status 30))
 (segment (start 219.014914 47.275086) (end 216.29 50) (width 0.25) (layer F.Cu) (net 3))
 (segment (start 250.885599 47.275086) (end 219.014914 47.275086) (width 0.25) (layer F.Cu) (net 3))
 (segment (start 256.160685 42) (end 250.885599 47.275086) (width 0.25) (layer F.Cu) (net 3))
 (segment (start 261.85034 42) (end 265 42) (width 0.5) (layer F.Cu) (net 2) (status 30))
 (segment (start 221.104904 47.725096) (end 218.83 50) (width 0.25) (layer F.Cu) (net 2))
 (segment (start 256.125244 47.725096) (end 221.104904 47.725096) (width 0.25) (layer F.Cu) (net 2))
 (segment (start 261.85034 42) (end 256.125244 47.725096) (width 0.25) (layer F.Cu) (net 2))
 (segment (start 267.54 42) (end 261.364894 48.175106) (width 0.25) (layer F.Cu) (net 1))
 (segment (start 223.194894 48.175106) (end 221.37 50) (width 0.25) (layer F.Cu) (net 1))
 (segment (start 261.364894 48.175106) (end 223.194894 48.175106) (width 0.25) (layer F.Cu) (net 1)))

